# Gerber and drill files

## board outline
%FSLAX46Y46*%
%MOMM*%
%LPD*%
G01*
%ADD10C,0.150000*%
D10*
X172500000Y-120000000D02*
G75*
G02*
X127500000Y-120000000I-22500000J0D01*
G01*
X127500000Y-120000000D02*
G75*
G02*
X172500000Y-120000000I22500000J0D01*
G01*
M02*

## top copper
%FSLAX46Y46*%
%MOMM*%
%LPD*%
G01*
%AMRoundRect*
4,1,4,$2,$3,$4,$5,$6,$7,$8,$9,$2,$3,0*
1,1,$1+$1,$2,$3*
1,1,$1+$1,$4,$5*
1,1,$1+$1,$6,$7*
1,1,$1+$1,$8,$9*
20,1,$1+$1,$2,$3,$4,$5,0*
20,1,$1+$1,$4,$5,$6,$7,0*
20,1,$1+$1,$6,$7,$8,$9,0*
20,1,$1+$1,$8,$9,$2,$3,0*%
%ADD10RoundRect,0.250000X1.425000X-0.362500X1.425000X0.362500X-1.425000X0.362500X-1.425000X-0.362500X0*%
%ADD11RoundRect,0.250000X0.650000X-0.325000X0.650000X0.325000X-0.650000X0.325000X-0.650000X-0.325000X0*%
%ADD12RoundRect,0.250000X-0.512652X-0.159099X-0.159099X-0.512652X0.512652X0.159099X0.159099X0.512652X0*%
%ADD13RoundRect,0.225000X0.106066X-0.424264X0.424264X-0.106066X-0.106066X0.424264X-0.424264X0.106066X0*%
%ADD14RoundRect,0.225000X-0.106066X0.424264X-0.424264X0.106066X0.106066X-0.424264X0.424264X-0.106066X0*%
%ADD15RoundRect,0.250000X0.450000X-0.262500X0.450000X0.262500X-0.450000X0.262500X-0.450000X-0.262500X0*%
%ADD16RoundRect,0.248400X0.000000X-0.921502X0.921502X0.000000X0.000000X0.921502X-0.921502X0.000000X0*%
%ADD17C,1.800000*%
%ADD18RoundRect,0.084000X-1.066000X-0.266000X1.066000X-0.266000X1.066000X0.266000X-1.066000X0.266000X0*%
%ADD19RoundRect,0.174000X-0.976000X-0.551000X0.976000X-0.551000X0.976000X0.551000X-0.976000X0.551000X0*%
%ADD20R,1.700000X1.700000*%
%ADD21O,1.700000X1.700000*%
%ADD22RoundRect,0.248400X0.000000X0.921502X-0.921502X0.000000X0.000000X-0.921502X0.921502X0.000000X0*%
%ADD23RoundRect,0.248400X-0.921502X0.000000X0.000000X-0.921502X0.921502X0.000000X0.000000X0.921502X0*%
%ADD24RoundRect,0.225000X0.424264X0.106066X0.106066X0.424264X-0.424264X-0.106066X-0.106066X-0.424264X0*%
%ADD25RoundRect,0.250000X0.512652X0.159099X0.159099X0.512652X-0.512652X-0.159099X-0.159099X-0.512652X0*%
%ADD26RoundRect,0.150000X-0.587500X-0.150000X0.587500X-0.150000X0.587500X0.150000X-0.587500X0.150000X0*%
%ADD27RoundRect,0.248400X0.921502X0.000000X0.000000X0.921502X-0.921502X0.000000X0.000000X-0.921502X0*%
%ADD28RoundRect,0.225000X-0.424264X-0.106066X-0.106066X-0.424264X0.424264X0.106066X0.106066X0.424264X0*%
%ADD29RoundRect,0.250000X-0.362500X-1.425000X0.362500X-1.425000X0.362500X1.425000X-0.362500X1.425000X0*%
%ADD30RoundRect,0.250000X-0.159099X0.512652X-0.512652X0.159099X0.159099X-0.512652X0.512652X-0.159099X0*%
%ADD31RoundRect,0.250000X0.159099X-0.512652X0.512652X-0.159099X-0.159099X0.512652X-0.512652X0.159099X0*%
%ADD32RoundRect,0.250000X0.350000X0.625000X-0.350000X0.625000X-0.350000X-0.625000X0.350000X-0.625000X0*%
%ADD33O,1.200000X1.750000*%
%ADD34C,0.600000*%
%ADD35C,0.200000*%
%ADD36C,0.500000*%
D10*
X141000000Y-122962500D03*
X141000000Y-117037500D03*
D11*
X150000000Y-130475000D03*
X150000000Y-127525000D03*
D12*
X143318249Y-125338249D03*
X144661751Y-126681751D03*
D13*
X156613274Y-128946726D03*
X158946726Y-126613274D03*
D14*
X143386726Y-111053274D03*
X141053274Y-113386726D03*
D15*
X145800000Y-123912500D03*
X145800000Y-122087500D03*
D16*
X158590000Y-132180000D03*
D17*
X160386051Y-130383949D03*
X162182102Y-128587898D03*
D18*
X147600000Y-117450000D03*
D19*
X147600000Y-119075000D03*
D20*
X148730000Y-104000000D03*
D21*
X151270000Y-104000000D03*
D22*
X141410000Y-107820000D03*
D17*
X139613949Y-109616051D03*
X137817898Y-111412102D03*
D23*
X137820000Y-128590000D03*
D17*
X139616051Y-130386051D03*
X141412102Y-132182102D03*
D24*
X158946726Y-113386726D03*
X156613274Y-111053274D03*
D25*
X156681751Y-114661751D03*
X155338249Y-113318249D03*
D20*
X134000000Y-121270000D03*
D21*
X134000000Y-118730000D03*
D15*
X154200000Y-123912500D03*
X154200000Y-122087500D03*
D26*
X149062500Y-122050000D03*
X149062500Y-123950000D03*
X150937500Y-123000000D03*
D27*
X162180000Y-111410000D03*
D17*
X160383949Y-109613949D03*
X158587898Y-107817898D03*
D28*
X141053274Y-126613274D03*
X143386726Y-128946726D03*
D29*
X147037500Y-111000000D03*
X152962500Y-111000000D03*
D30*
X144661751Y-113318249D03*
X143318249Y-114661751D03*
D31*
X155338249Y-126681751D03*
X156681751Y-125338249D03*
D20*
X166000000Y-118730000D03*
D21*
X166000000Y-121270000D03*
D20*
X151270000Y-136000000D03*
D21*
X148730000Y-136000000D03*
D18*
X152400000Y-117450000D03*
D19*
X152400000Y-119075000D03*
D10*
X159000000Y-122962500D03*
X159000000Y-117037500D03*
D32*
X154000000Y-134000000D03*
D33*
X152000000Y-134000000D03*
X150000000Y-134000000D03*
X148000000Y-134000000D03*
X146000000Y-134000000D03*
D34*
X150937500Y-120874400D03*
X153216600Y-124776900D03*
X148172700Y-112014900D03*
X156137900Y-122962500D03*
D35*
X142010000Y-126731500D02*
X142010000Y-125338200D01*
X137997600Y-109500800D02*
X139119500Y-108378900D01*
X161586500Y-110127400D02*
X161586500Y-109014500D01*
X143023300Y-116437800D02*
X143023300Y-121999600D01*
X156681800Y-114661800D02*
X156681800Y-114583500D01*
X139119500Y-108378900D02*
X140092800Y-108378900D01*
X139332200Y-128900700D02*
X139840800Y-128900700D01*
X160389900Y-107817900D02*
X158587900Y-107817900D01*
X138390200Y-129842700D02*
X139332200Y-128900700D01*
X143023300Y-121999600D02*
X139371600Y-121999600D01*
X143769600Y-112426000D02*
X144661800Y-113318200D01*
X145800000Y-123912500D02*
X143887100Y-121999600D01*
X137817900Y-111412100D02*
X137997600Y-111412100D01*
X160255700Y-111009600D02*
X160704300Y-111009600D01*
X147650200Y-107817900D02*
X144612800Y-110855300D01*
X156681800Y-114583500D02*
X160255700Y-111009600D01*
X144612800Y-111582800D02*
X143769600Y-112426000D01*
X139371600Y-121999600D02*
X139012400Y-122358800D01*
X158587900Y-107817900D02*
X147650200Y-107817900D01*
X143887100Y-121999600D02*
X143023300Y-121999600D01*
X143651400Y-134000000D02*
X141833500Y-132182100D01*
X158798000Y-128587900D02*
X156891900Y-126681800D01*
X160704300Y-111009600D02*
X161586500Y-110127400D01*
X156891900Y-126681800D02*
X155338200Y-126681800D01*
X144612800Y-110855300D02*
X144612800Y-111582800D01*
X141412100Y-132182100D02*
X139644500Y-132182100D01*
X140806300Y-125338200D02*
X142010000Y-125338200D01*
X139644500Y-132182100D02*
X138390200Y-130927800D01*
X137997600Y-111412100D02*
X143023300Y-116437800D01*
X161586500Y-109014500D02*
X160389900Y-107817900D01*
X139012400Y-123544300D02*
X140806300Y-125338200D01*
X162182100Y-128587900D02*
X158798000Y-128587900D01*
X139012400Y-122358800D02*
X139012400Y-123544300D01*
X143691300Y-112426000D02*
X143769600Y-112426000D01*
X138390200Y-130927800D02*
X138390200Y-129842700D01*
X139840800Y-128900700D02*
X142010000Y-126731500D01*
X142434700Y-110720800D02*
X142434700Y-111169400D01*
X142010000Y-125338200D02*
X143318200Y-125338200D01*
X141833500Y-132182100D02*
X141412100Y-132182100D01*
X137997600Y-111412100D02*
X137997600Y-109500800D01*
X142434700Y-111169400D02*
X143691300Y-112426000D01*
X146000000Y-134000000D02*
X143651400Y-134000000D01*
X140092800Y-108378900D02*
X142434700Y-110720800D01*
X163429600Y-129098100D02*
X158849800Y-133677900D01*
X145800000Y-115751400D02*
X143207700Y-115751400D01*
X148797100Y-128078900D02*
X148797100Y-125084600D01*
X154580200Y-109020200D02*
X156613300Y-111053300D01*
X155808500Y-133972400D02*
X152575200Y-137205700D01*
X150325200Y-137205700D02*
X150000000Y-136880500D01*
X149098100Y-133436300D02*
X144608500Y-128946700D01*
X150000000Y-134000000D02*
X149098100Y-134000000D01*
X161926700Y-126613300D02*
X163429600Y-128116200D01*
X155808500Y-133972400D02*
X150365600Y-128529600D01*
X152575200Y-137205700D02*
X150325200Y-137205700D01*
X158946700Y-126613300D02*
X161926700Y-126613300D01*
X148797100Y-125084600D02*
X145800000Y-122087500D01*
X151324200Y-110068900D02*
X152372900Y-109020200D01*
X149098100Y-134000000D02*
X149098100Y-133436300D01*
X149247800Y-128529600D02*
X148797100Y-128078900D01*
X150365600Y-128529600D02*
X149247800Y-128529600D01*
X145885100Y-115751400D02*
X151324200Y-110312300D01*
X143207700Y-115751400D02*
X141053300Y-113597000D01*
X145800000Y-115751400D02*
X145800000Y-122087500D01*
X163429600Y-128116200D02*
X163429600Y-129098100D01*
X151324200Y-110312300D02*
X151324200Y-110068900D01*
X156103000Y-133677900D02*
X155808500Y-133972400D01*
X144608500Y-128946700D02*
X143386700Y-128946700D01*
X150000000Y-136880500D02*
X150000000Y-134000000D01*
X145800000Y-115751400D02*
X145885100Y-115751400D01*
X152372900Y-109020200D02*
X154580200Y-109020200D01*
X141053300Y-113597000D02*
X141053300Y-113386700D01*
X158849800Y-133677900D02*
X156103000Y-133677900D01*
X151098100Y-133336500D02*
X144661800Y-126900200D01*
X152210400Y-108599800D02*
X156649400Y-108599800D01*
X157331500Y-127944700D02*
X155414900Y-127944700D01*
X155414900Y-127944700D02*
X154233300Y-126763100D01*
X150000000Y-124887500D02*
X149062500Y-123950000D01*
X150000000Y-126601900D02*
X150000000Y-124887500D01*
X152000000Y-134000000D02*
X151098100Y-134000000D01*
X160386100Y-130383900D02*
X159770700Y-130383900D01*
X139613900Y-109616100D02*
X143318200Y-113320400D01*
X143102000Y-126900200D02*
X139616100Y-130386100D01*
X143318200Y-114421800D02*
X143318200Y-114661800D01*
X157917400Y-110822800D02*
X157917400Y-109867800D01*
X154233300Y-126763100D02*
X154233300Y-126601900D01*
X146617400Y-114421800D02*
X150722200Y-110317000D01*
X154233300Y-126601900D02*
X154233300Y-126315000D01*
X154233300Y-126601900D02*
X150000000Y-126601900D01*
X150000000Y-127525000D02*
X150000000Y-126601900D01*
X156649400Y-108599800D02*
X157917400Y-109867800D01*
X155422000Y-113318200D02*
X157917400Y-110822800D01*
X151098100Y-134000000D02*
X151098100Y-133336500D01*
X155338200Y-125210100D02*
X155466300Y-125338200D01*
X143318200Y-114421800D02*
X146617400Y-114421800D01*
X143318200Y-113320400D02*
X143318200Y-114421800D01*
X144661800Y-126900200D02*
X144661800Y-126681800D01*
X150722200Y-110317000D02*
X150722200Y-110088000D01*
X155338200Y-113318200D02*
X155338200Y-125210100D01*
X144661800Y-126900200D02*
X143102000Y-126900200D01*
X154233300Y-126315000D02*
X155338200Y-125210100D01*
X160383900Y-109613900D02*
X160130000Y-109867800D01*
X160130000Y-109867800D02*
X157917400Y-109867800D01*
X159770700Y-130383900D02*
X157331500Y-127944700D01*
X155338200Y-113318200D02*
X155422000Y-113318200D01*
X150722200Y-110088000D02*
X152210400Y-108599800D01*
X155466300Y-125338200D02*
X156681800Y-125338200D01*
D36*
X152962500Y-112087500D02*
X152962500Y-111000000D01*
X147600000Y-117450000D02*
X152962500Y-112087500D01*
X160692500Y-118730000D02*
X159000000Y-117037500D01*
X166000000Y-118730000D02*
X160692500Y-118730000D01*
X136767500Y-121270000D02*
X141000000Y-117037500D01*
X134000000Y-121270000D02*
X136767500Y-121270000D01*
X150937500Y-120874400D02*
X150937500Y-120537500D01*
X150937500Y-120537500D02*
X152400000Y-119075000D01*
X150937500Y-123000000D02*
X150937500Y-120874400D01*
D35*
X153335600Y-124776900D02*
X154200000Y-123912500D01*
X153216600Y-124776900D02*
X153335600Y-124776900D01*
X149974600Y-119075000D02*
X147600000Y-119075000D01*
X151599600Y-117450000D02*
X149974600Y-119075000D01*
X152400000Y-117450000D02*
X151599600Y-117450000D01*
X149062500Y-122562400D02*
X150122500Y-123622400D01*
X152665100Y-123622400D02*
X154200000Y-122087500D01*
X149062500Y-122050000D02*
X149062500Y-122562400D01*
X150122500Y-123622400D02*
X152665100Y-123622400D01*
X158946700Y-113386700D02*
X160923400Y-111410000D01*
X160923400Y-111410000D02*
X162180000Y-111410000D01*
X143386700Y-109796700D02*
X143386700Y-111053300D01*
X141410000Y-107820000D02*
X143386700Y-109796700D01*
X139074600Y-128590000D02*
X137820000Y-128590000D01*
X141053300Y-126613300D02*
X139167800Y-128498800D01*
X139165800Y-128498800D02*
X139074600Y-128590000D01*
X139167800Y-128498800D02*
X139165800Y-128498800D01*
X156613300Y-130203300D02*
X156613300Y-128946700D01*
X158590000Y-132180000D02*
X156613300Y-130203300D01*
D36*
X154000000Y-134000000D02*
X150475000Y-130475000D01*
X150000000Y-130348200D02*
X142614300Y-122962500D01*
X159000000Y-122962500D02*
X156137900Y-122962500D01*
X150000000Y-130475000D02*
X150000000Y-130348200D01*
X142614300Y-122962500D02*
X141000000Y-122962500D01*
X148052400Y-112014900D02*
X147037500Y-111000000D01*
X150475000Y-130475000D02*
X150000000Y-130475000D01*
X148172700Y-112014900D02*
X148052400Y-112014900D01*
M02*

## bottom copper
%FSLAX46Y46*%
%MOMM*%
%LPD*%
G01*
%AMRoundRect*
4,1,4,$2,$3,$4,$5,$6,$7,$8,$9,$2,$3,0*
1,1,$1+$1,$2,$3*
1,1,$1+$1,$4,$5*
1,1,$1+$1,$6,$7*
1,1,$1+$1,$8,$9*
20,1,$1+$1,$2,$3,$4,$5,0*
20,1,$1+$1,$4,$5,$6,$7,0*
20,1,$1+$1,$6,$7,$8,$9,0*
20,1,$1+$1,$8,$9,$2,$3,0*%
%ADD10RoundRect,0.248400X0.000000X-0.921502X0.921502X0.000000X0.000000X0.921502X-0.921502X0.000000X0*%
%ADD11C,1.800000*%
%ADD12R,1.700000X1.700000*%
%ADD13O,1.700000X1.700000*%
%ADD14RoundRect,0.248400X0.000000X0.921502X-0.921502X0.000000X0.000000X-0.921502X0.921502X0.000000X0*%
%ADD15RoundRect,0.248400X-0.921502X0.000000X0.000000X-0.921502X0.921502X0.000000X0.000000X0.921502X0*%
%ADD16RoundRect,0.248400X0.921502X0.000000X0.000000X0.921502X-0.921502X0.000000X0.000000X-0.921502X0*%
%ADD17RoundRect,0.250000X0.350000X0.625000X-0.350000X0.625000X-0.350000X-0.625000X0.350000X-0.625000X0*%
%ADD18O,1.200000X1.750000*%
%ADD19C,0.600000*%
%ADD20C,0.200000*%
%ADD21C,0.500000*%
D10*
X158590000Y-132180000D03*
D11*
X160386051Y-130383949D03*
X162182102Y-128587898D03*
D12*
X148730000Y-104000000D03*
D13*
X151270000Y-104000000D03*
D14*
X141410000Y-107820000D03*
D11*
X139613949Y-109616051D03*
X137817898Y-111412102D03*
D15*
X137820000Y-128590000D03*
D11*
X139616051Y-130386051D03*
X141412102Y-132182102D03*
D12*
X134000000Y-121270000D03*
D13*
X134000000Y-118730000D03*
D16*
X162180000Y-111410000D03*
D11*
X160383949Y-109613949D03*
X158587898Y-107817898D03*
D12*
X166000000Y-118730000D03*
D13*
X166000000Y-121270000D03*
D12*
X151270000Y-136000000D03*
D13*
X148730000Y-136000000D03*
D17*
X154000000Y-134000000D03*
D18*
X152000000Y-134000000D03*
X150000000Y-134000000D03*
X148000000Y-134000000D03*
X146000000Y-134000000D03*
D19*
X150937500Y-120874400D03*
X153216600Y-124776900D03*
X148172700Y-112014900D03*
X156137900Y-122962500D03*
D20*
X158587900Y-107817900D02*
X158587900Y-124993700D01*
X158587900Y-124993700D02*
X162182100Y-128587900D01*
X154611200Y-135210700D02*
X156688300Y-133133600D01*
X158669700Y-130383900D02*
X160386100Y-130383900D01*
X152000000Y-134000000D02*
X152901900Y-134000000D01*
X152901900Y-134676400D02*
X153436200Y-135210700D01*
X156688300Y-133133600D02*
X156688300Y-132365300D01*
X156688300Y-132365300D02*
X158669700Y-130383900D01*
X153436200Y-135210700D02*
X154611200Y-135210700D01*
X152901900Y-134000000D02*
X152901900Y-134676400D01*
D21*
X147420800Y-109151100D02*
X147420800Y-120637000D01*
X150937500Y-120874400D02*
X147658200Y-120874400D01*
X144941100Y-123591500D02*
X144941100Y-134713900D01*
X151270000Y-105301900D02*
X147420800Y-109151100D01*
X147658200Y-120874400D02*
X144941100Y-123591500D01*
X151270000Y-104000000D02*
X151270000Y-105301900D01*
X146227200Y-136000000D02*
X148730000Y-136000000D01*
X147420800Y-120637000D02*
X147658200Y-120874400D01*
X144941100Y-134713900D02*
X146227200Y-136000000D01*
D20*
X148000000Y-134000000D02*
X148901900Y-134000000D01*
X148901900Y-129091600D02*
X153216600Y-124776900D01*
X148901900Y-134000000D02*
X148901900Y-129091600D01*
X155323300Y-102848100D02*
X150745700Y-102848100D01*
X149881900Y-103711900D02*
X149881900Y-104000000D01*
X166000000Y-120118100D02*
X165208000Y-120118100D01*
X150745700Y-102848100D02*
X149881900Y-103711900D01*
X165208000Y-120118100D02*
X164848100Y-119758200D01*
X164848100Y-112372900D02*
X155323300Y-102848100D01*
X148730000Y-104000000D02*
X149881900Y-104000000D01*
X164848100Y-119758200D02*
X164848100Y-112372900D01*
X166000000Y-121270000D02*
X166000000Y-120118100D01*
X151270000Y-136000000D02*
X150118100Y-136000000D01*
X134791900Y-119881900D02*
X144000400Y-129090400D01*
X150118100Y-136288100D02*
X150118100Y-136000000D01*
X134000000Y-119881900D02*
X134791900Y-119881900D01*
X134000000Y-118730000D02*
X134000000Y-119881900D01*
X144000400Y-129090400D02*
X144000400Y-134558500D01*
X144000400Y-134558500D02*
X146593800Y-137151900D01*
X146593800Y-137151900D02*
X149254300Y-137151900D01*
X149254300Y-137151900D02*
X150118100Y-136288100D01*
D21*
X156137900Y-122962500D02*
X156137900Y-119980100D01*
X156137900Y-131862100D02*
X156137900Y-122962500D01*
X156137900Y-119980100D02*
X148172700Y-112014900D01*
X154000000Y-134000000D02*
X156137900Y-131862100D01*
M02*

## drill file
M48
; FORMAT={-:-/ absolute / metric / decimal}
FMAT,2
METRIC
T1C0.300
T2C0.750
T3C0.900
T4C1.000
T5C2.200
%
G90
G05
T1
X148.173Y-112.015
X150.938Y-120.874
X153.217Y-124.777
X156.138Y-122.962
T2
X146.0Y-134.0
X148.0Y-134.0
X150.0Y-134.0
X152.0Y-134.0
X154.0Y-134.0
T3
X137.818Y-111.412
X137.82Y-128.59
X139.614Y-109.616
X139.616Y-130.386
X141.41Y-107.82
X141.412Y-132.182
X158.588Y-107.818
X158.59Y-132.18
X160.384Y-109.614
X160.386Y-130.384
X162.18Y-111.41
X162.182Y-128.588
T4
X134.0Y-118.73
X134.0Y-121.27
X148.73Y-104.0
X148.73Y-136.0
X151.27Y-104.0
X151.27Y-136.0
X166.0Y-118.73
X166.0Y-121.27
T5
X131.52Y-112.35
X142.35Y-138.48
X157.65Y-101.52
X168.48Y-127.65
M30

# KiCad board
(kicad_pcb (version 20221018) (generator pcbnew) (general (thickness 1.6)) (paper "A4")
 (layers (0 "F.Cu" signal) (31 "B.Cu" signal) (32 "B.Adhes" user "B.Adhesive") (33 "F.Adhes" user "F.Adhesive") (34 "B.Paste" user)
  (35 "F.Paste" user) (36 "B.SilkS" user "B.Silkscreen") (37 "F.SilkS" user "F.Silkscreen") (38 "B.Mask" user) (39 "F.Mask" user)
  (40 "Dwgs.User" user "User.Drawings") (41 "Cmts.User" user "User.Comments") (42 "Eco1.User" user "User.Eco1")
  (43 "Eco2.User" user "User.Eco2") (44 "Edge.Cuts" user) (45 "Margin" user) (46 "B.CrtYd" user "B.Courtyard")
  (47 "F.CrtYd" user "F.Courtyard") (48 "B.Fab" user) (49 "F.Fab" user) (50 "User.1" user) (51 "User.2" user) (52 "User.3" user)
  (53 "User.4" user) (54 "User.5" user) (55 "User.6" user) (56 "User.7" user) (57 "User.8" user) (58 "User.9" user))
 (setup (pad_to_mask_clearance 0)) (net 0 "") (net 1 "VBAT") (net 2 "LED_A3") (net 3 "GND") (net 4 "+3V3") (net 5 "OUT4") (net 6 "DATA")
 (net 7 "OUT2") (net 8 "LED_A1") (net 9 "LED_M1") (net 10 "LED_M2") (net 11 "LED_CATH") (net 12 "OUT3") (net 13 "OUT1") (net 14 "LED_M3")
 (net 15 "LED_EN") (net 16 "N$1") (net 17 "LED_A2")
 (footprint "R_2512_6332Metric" (layer "F.Cu") (at 141 120 90)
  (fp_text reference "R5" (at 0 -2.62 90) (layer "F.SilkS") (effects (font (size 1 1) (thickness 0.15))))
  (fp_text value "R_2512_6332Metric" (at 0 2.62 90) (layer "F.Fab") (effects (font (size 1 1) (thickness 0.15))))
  (pad "1" smd roundrect (at -2.9625 0 90) (size 1.225 3.35) (layers "F.Cu" "F.Paste" "F.Mask") (roundrect_rratio 0.204082) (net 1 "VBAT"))
  (pad "2" smd roundrect (at 2.9625 0 90) (size 1.225 3.35) (layers "F.Cu" "F.Paste" "F.Mask") (roundrect_rratio 0.204082) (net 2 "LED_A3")))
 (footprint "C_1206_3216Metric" (layer "F.Cu") (at 150 129 90)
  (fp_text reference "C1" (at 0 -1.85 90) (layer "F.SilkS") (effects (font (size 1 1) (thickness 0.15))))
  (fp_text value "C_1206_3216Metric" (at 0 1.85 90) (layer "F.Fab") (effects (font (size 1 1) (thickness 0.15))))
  (pad "1" smd roundrect (at -1.475 0 90) (size 1.15 1.8) (layers "F.Cu" "F.Paste" "F.Mask") (roundrect_rratio 0.217391) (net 1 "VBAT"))
  (pad "2" smd roundrect (at 1.475 0 90) (size 1.15 1.8) (layers "F.Cu" "F.Paste" "F.Mask") (roundrect_rratio 0.217391) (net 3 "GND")))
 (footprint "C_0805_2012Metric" (layer "F.Cu") (at 143.99 126.01 -45)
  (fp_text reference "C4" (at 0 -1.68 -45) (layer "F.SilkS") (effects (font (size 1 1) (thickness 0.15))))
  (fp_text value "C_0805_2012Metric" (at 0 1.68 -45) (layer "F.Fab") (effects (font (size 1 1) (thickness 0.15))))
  (pad "1" smd roundrect (at -0.95 0 315) (size 1 1.45) (layers "F.Cu" "F.Paste" "F.Mask") (roundrect_rratio 0.25) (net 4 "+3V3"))
  (pad "2" smd roundrect (at 0.95 0 315) (size 1 1.45) (layers "F.Cu" "F.Paste" "F.Mask") (roundrect_rratio 0.25) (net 3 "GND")))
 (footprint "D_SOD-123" (layer "F.Cu") (at 157.78 127.78 45)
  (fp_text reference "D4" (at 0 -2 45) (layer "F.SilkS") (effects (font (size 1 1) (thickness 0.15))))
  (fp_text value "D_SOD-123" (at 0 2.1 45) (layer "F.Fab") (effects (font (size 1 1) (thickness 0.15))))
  (pad "1" smd roundrect (at -1.65 0 45) (size 0.9 1.2) (layers "F.Cu" "F.Paste" "F.Mask") (roundrect_rratio 0.25) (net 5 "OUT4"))
  (pad "2" smd roundrect (at 1.65 0 45) (size 0.9 1.2) (layers "F.Cu" "F.Paste" "F.Mask") (roundrect_rratio 0.25) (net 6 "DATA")))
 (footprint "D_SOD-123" (layer "F.Cu") (at 142.22 112.22 -135)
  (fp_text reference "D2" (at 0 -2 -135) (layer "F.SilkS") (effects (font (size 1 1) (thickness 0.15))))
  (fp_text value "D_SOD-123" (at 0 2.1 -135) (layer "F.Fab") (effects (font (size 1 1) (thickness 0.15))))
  (pad "1" smd roundrect (at -1.65 0 225) (size 0.9 1.2) (layers "F.Cu" "F.Paste" "F.Mask") (roundrect_rratio 0.25) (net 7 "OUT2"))
  (pad "2" smd roundrect (at 1.65 0 225) (size 0.9 1.2) (layers "F.Cu" "F.Paste" "F.Mask") (roundrect_rratio 0.25) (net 6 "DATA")))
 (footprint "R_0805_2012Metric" (layer "F.Cu") (at 145.8 123 90)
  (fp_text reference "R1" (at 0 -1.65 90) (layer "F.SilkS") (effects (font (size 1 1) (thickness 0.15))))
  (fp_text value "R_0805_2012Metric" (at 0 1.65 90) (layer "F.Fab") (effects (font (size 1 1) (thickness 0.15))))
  (pad "1" smd roundrect (at -0.9125 0 90) (size 1.025 1.4) (layers "F.Cu" "F.Paste" "F.Mask") (roundrect_rratio 0.243902) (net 4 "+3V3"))
  (pad "2" smd roundrect (at 0.9125 0 90) (size 1.025 1.4) (layers "F.Cu" "F.Paste" "F.Mask") (roundrect_rratio 0.243902) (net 6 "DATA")))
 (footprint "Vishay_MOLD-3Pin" (layer "F.Cu") (at 158.59 132.18 45)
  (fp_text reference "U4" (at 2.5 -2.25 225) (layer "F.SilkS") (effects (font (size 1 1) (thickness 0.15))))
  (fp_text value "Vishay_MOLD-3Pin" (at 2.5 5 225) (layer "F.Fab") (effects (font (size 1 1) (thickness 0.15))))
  (pad "1" thru_hole roundrect (at 0 0 45) (size 1.8 1.8) (drill 0.9) (layers "*.Cu" "*.Mask") (roundrect_rratio 0.138) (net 5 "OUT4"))
  (pad "2" thru_hole circle (at 2.54 0 45) (size 1.8 1.8) (drill 0.9) (layers "*.Cu" "*.Mask") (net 3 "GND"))
  (pad "3" thru_hole circle (at 5.08 0 45) (size 1.8 1.8) (drill 0.9) (layers "*.Cu" "*.Mask") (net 4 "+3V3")))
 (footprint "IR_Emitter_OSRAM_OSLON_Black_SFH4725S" (layer "F.Cu") (at 147.6 118.5)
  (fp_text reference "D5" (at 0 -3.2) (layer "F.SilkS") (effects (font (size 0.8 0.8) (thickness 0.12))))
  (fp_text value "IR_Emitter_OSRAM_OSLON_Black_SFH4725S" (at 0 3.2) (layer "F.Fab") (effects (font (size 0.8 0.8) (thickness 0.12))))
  (pad "1" smd roundrect (at 0 -1.05) (size 2.3 0.7) (layers "F.Cu" "F.Paste" "F.Mask") (roundrect_rratio 0.12) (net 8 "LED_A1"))
  (pad "2" smd roundrect (at 0 0.575) (size 2.3 1.45) (layers "F.Cu" "F.Paste" "F.Mask") (roundrect_rratio 0.12) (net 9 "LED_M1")))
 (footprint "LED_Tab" (layer "F.Cu") (at 148.73 104 90)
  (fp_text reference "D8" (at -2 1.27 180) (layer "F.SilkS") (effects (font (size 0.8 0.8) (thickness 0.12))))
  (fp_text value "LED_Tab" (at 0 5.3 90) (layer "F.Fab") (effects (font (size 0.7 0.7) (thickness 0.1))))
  (pad "1" thru_hole rect (at 0 0 90) (size 1.7 1.7) (drill 1) (layers "*.Cu" "*.Mask") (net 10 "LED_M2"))
  (pad "2" thru_hole oval (at 0 2.54 90) (size 1.7 1.7) (drill 1) (layers "*.Cu" "*.Mask") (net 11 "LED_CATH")))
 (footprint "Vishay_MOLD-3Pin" (layer "F.Cu") (at 141.41 107.82 -135)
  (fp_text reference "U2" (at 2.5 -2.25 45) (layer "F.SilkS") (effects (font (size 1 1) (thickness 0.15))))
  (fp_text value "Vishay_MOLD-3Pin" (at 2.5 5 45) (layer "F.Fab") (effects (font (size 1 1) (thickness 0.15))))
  (pad "1" thru_hole roundrect (at 0 0 225) (size 1.8 1.8) (drill 0.9) (layers "*.Cu" "*.Mask") (roundrect_rratio 0.138) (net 7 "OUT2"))
  (pad "2" thru_hole circle (at 2.54 0 225) (size 1.8 1.8) (drill 0.9) (layers "*.Cu" "*.Mask") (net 3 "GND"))
  (pad "3" thru_hole circle (at 5.08 0 225) (size 1.8 1.8) (drill 0.9) (layers "*.Cu" "*.Mask") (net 4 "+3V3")))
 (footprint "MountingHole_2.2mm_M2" (layer "F.Cu") (at 131.52 112.35)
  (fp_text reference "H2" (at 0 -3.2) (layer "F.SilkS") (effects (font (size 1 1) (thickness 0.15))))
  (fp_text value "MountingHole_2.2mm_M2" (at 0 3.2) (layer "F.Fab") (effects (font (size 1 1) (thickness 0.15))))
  (pad "" np_thru_hole circle (at 0 0) (size 2.2 2.2) (drill 2.2) (layers "*.Cu" "*.Mask")))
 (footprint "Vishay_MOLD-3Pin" (layer "F.Cu") (at 137.82 128.59 -45)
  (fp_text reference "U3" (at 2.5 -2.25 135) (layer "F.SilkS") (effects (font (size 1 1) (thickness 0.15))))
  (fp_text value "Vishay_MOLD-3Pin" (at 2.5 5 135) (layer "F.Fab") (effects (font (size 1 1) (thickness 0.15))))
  (pad "1" thru_hole roundrect (at 0 0 315) (size 1.8 1.8) (drill 0.9) (layers "*.Cu" "*.Mask") (roundrect_rratio 0.138) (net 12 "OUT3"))
  (pad "2" thru_hole circle (at 2.54 0 315) (size 1.8 1.8) (drill 0.9) (layers "*.Cu" "*.Mask") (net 3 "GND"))
  (pad "3" thru_hole circle (at 5.08 0 315) (size 1.8 1.8) (drill 0.9) (layers "*.Cu" "*.Mask") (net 4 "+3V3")))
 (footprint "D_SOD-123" (layer "F.Cu") (at 157.78 112.22 135)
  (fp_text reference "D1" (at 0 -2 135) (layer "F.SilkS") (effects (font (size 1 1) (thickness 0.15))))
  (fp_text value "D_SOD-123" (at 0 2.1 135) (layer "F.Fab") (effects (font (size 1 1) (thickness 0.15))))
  (pad "1" smd roundrect (at -1.65 0 135) (size 0.9 1.2) (layers "F.Cu" "F.Paste" "F.Mask") (roundrect_rratio 0.25) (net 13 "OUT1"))
  (pad "2" smd roundrect (at 1.65 0 135) (size 0.9 1.2) (layers "F.Cu" "F.Paste" "F.Mask") (roundrect_rratio 0.25) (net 6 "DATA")))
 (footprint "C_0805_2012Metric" (layer "F.Cu") (at 156.01 113.99 135)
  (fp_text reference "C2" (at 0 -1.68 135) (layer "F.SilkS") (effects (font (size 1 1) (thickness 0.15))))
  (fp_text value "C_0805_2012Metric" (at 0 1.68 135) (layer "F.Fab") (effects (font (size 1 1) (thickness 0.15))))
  (pad "1" smd roundrect (at -0.95 0 135) (size 1 1.45) (layers "F.Cu" "F.Paste" "F.Mask") (roundrect_rratio 0.25) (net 4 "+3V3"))
  (pad "2" smd roundrect (at 0.95 0 135) (size 1 1.45) (layers "F.Cu" "F.Paste" "F.Mask") (roundrect_rratio 0.25) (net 3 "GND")))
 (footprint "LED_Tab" (layer "F.Cu") (at 134 121.27 180)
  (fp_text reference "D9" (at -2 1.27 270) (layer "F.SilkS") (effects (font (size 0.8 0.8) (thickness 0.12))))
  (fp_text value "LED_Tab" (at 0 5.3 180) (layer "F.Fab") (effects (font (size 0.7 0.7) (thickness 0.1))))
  (pad "1" thru_hole rect (at 0 0 180) (size 1.7 1.7) (drill 1) (layers "*.Cu" "*.Mask") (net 2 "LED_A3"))
  (pad "2" thru_hole oval (at 0 2.54 180) (size 1.7 1.7) (drill 1) (layers "*.Cu" "*.Mask") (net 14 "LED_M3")))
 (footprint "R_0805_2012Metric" (layer "F.Cu") (at 154.2 123 90)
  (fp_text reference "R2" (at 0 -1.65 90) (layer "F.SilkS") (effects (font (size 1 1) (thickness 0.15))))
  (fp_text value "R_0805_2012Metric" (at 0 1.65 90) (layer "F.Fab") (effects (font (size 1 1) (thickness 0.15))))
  (pad "1" smd roundrect (at -0.9125 0 90) (size 1.025 1.4) (layers "F.Cu" "F.Paste" "F.Mask") (roundrect_rratio 0.243902) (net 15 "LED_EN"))
  (pad "2" smd roundrect (at 0.9125 0 90) (size 1.025 1.4) (layers "F.Cu" "F.Paste" "F.Mask") (roundrect_rratio 0.243902) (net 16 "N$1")))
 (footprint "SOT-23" (layer "F.Cu") (at 150 123)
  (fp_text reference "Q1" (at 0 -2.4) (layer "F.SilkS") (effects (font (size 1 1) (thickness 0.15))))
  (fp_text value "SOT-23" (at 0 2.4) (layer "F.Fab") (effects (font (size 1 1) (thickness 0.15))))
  (pad "1" smd roundrect (at -0.9375 -0.95) (size 1.475 0.6) (layers "F.Cu" "F.Paste" "F.Mask") (roundrect_rratio 0.25) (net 16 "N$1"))
  (pad "2" smd roundrect (at -0.9375 0.95) (size 1.475 0.6) (layers "F.Cu" "F.Paste" "F.Mask") (roundrect_rratio 0.25) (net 3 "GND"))
  (pad "3" smd roundrect (at 0.9375 0) (size 1.475 0.6) (layers "F.Cu" "F.Paste" "F.Mask") (roundrect_rratio 0.25) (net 11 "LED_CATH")))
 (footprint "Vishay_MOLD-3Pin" (layer "F.Cu") (at 162.18 111.41 135)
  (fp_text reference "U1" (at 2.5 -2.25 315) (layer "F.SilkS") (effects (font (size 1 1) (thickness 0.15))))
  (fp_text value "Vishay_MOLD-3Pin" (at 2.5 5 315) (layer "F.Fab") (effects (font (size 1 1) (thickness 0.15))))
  (pad "1" thru_hole roundrect (at 0 0 135) (size 1.8 1.8) (drill 0.9) (layers "*.Cu" "*.Mask") (roundrect_rratio 0.138) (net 13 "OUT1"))
  (pad "2" thru_hole circle (at 2.54 0 135) (size 1.8 1.8) (drill 0.9) (layers "*.Cu" "*.Mask") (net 3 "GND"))
  (pad "3" thru_hole circle (at 5.08 0 135) (size 1.8 1.8) (drill 0.9) (layers "*.Cu" "*.Mask") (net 4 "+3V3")))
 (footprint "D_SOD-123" (layer "F.Cu") (at 142.22 127.78 -45)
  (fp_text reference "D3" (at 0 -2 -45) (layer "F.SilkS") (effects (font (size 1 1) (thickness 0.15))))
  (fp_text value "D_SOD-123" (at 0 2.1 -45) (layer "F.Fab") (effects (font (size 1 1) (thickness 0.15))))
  (pad "1" smd roundrect (at -1.65 0 315) (size 0.9 1.2) (layers "F.Cu" "F.Paste" "F.Mask") (roundrect_rratio 0.25) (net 12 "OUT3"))
  (pad "2" smd roundrect (at 1.65 0 315) (size 0.9 1.2) (layers "F.Cu" "F.Paste" "F.Mask") (roundrect_rratio 0.25) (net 6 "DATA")))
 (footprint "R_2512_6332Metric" (layer "F.Cu") (at 150 111)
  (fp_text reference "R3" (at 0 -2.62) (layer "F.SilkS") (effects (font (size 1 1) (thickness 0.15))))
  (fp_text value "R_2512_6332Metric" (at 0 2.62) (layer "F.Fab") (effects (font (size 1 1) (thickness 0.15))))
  (pad "1" smd roundrect (at -2.9625 0) (size 1.225 3.35) (layers "F.Cu" "F.Paste" "F.Mask") (roundrect_rratio 0.204082) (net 1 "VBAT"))
  (pad "2" smd roundrect (at 2.9625 0) (size 1.225 3.35) (layers "F.Cu" "F.Paste" "F.Mask") (roundrect_rratio 0.204082) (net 8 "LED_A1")))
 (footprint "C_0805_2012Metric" (layer "F.Cu") (at 143.99 113.99 -135)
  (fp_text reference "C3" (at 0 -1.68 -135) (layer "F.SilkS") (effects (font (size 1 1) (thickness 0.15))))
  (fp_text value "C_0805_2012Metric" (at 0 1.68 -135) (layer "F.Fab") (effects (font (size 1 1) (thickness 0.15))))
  (pad "1" smd roundrect (at -0.95 0 225) (size 1 1.45) (layers "F.Cu" "F.Paste" "F.Mask") (roundrect_rratio 0.25) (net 4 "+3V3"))
  (pad "2" smd roundrect (at 0.95 0 225) (size 1 1.45) (layers "F.Cu" "F.Paste" "F.Mask") (roundrect_rratio 0.25) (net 3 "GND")))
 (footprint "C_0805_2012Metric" (layer "F.Cu") (at 156.01 126.01 45)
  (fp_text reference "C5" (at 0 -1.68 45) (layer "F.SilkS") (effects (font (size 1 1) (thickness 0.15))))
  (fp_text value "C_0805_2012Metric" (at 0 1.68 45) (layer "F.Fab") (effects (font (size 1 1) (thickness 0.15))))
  (pad "1" smd roundrect (at -0.95 0 45) (size 1 1.45) (layers "F.Cu" "F.Paste" "F.Mask") (roundrect_rratio 0.25) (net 4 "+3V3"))
  (pad "2" smd roundrect (at 0.95 0 45) (size 1 1.45) (layers "F.Cu" "F.Paste" "F.Mask") (roundrect_rratio 0.25) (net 3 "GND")))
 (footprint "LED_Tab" (layer "F.Cu") (at 166 118.73)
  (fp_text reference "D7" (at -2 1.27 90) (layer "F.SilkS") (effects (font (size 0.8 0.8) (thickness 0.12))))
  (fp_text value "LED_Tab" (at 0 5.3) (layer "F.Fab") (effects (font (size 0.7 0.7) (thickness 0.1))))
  (pad "1" thru_hole rect (at 0 0) (size 1.7 1.7) (drill 1) (layers "*.Cu" "*.Mask") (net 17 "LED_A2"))
  (pad "2" thru_hole oval (at 0 2.54) (size 1.7 1.7) (drill 1) (layers "*.Cu" "*.Mask") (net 10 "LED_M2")))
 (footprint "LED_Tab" (layer "F.Cu") (at 151.27 136 -90)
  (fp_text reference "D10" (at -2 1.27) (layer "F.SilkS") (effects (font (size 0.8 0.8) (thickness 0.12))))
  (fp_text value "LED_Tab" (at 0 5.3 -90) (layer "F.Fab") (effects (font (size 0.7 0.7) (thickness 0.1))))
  (pad "1" thru_hole rect (at 0 0 270) (size 1.7 1.7) (drill 1) (layers "*.Cu" "*.Mask") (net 14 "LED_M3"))
  (pad "2" thru_hole oval (at 0 2.54 270) (size 1.7 1.7) (drill 1) (layers "*.Cu" "*.Mask") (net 11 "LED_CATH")))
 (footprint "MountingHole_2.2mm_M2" (layer "F.Cu") (at 168.48 127.65)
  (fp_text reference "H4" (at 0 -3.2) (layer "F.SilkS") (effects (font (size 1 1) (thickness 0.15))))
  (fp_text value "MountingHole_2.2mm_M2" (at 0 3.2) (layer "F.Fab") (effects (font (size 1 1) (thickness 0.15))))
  (pad "" np_thru_hole circle (at 0 0) (size 2.2 2.2) (drill 2.2) (layers "*.Cu" "*.Mask")))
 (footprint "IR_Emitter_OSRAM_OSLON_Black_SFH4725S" (layer "F.Cu") (at 152.4 118.5)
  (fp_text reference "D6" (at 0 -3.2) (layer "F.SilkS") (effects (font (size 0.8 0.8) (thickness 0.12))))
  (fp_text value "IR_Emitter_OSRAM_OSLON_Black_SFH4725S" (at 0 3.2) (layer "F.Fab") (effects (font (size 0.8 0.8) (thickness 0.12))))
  (pad "1" smd roundrect (at 0 -1.05) (size 2.3 0.7) (layers "F.Cu" "F.Paste" "F.Mask") (roundrect_rratio 0.12) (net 9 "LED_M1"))
  (pad "2" smd roundrect (at 0 0.575) (size 2.3 1.45) (layers "F.Cu" "F.Paste" "F.Mask") (roundrect_rratio 0.12) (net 11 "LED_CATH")))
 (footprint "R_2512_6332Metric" (layer "F.Cu") (at 159 120 90)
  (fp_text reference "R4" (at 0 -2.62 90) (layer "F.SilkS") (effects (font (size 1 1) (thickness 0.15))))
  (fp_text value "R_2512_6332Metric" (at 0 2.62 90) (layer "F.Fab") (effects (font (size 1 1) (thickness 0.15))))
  (pad "1" smd roundrect (at -2.9625 0 90) (size 1.225 3.35) (layers "F.Cu" "F.Paste" "F.Mask") (roundrect_rratio 0.204082) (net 1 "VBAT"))
  (pad "2" smd roundrect (at 2.9625 0 90) (size 1.225 3.35) (layers "F.Cu" "F.Paste" "F.Mask") (roundrect_rratio 0.204082) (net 17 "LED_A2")))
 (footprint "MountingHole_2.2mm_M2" (layer "F.Cu") (at 142.35 138.48)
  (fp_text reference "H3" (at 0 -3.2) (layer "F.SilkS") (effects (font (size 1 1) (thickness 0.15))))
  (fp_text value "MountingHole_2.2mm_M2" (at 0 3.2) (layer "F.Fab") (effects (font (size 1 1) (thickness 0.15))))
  (pad "" np_thru_hole circle (at 0 0) (size 2.2 2.2) (drill 2.2) (layers "*.Cu" "*.Mask")))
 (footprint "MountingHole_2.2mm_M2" (layer "F.Cu") (at 157.65 101.52)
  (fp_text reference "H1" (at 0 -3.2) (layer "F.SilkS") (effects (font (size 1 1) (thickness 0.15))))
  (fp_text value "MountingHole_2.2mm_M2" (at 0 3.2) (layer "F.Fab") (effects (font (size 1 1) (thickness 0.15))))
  (pad "" np_thru_hole circle (at 0 0) (size 2.2 2.2) (drill 2.2) (layers "*.Cu" "*.Mask")))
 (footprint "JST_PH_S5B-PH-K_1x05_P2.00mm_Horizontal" (layer "B.Cu") (at 154 134 180)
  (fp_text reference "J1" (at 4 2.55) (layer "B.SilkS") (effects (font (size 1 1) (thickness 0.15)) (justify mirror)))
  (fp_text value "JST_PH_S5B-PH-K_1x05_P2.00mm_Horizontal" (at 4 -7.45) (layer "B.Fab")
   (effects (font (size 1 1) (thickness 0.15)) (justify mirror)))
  (pad "1" thru_hole roundrect (at 0 0 180) (size 1.2 1.75) (drill 0.75) (layers "*.Cu" "*.Mask") (roundrect_rratio 0.208333) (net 1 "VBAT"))
  (pad "2" thru_hole oval (at 2 0 180) (size 1.2 1.75) (drill 0.75) (layers "*.Cu" "*.Mask") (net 3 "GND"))
  (pad "3" thru_hole oval (at 4 0 180) (size 1.2 1.75) (drill 0.75) (layers "*.Cu" "*.Mask") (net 6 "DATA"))
  (pad "4" thru_hole oval (at 6 0 180) (size 1.2 1.75) (drill 0.75) (layers "*.Cu" "*.Mask") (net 15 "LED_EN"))
  (pad "5" thru_hole oval (at 8 0 180) (size 1.2 1.75) (drill 0.75) (layers "*.Cu" "*.Mask") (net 4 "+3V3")))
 (gr_circle (center 150 120) (end 172.5 120) (stroke (width 0.15) (type default)) (fill none) (layer "Edge.Cuts"))
 (segment (start 142.01 126.7315) (end 142.01 125.3382) (width 0.2) (layer "F.Cu") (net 4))
 (segment (start 137.9976 109.5008) (end 139.1195 108.3789) (width 0.2) (layer "F.Cu") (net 4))
 (segment (start 161.5865 110.1274) (end 161.5865 109.0145) (width 0.2) (layer "F.Cu") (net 4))
 (segment (start 143.0233 116.4378) (end 143.0233 121.9996) (width 0.2) (layer "F.Cu") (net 4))
 (segment (start 156.6818 114.6618) (end 156.6818 114.5835) (width 0.2) (layer "F.Cu") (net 4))
 (segment (start 139.1195 108.3789) (end 140.0928 108.3789) (width 0.2) (layer "F.Cu") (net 4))
 (segment (start 139.3322 128.9007) (end 139.8408 128.9007) (width 0.2) (layer "F.Cu") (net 4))
 (segment (start 160.3899 107.8179) (end 158.5879 107.8179) (width 0.2) (layer "F.Cu") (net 4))
 (segment (start 138.3902 129.8427) (end 139.3322 128.9007) (width 0.2) (layer "F.Cu") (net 4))
 (segment (start 143.0233 121.9996) (end 139.3716 121.9996) (width 0.2) (layer "F.Cu") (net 4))
 (segment (start 143.7696 112.426) (end 144.6618 113.3182) (width 0.2) (layer "F.Cu") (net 4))
 (segment (start 145.8 123.9125) (end 143.8871 121.9996) (width 0.2) (layer "F.Cu") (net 4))
 (segment (start 137.8179 111.4121) (end 137.9976 111.4121) (width 0.2) (layer "F.Cu") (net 4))
 (segment (start 160.2557 111.0096) (end 160.7043 111.0096) (width 0.2) (layer "F.Cu") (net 4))
 (segment (start 147.6502 107.8179) (end 144.6128 110.8553) (width 0.2) (layer "F.Cu") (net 4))
 (segment (start 156.6818 114.5835) (end 160.2557 111.0096) (width 0.2) (layer "F.Cu") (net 4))
 (segment (start 144.6128 111.5828) (end 143.7696 112.426) (width 0.2) (layer "F.Cu") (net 4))
 (segment (start 139.3716 121.9996) (end 139.0124 122.3588) (width 0.2) (layer "F.Cu") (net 4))
 (segment (start 158.5879 107.8179) (end 147.6502 107.8179) (width 0.2) (layer "F.Cu") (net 4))
 (segment (start 143.8871 121.9996) (end 143.0233 121.9996) (width 0.2) (layer "F.Cu") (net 4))
 (segment (start 143.6514 134) (end 141.8335 132.1821) (width 0.2) (layer "F.Cu") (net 4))
 (segment (start 158.798 128.5879) (end 156.8919 126.6818) (width 0.2) (layer "F.Cu") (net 4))
 (segment (start 160.7043 111.0096) (end 161.5865 110.1274) (width 0.2) (layer "F.Cu") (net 4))
 (segment (start 156.8919 126.6818) (end 155.3382 126.6818) (width 0.2) (layer "F.Cu") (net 4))
 (segment (start 144.6128 110.8553) (end 144.6128 111.5828) (width 0.2) (layer "F.Cu") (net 4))
 (segment (start 141.4121 132.1821) (end 139.6445 132.1821) (width 0.2) (layer "F.Cu") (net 4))
 (segment (start 140.8063 125.3382) (end 142.01 125.3382) (width 0.2) (layer "F.Cu") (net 4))
 (segment (start 139.6445 132.1821) (end 138.3902 130.9278) (width 0.2) (layer "F.Cu") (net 4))
 (segment (start 137.9976 111.4121) (end 143.0233 116.4378) (width 0.2) (layer "F.Cu") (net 4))
 (segment (start 161.5865 109.0145) (end 160.3899 107.8179) (width 0.2) (layer "F.Cu") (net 4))
 (segment (start 139.0124 123.5443) (end 140.8063 125.3382) (width 0.2) (layer "F.Cu") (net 4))
 (segment (start 162.1821 128.5879) (end 158.798 128.5879) (width 0.2) (layer "F.Cu") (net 4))
 (segment (start 139.0124 122.3588) (end 139.0124 123.5443) (width 0.2) (layer "F.Cu") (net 4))
 (segment (start 143.6913 112.426) (end 143.7696 112.426) (width 0.2) (layer "F.Cu") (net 4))
 (segment (start 138.3902 130.9278) (end 138.3902 129.8427) (width 0.2) (layer "F.Cu") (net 4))
 (segment (start 139.8408 128.9007) (end 142.01 126.7315) (width 0.2) (layer "F.Cu") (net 4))
 (segment (start 142.4347 110.7208) (end 142.4347 111.1694) (width 0.2) (layer "F.Cu") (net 4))
 (segment (start 142.01 125.3382) (end 143.3182 125.3382) (width 0.2) (layer "F.Cu") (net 4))
 (segment (start 141.8335 132.1821) (end 141.4121 132.1821) (width 0.2) (layer "F.Cu") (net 4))
 (segment (start 137.9976 111.4121) (end 137.9976 109.5008) (width 0.2) (layer "F.Cu") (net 4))
 (segment (start 142.4347 111.1694) (end 143.6913 112.426) (width 0.2) (layer "F.Cu") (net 4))
 (segment (start 146 134) (end 143.6514 134) (width 0.2) (layer "F.Cu") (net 4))
 (segment (start 140.0928 108.3789) (end 142.4347 110.7208) (width 0.2) (layer "F.Cu") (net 4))
 (segment (start 158.5879 107.8179) (end 158.5879 124.9937) (width 0.2) (layer "B.Cu") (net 4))
 (segment (start 158.5879 124.9937) (end 162.1821 128.5879) (width 0.2) (layer "B.Cu") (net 4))
 (segment (start 163.4296 129.0981) (end 158.8498 133.6779) (width 0.2) (layer "F.Cu") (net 6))
 (segment (start 145.8 115.7514) (end 143.2077 115.7514) (width 0.2) (layer "F.Cu") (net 6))
 (segment (start 148.7971 128.0789) (end 148.7971 125.0846) (width 0.2) (layer "F.Cu") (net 6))
 (segment (start 154.5802 109.0202) (end 156.6133 111.0533) (width 0.2) (layer "F.Cu") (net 6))
 (segment (start 155.8085 133.9724) (end 152.5752 137.2057) (width 0.2) (layer "F.Cu") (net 6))
 (segment (start 150.3252 137.2057) (end 150 136.8805) (width 0.2) (layer "F.Cu") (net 6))
 (segment (start 149.0981 133.4363) (end 144.6085 128.9467) (width 0.2) (layer "F.Cu") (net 6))
 (segment (start 150 134) (end 149.0981 134) (width 0.2) (layer "F.Cu") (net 6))
 (segment (start 161.9267 126.6133) (end 163.4296 128.1162) (width 0.2) (layer "F.Cu") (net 6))
 (segment (start 155.8085 133.9724) (end 150.3656 128.5296) (width 0.2) (layer "F.Cu") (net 6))
 (segment (start 152.5752 137.2057) (end 150.3252 137.2057) (width 0.2) (layer "F.Cu") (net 6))
 (segment (start 158.9467 126.6133) (end 161.9267 126.6133) (width 0.2) (layer "F.Cu") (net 6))
 (segment (start 148.7971 125.0846) (end 145.8 122.0875) (width 0.2) (layer "F.Cu") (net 6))
 (segment (start 151.3242 110.0689) (end 152.3729 109.0202) (width 0.2) (layer "F.Cu") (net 6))
 (segment (start 149.0981 134) (end 149.0981 133.4363) (width 0.2) (layer "F.Cu") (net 6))
 (segment (start 149.2478 128.5296) (end 148.7971 128.0789) (width 0.2) (layer "F.Cu") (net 6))
 (segment (start 150.3656 128.5296) (end 149.2478 128.5296) (width 0.2) (layer "F.Cu") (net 6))
 (segment (start 145.8851 115.7514) (end 151.3242 110.3123) (width 0.2) (layer "F.Cu") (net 6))
 (segment (start 143.2077 115.7514) (end 141.0533 113.597) (width 0.2) (layer "F.Cu") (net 6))
 (segment (start 145.8 115.7514) (end 145.8 122.0875) (width 0.2) (layer "F.Cu") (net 6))
 (segment (start 163.4296 128.1162) (end 163.4296 129.0981) (width 0.2) (layer "F.Cu") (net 6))
 (segment (start 151.3242 110.3123) (end 151.3242 110.0689) (width 0.2) (layer "F.Cu") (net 6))
 (segment (start 156.103 133.6779) (end 155.8085 133.9724) (width 0.2) (layer "F.Cu") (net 6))
 (segment (start 144.6085 128.9467) (end 143.3867 128.9467) (width 0.2) (layer "F.Cu") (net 6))
 (segment (start 150 136.8805) (end 150 134) (width 0.2) (layer "F.Cu") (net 6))
 (segment (start 145.8 115.7514) (end 145.8851 115.7514) (width 0.2) (layer "F.Cu") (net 6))
 (segment (start 152.3729 109.0202) (end 154.5802 109.0202) (width 0.2) (layer "F.Cu") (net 6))
 (segment (start 141.0533 113.597) (end 141.0533 113.3867) (width 0.2) (layer "F.Cu") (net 6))
 (segment (start 158.8498 133.6779) (end 156.103 133.6779) (width 0.2) (layer "F.Cu") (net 6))
 (segment (start 151.0981 133.3365) (end 144.6618 126.9002) (width 0.2) (layer "F.Cu") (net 3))
 (segment (start 152.2104 108.5998) (end 156.6494 108.5998) (width 0.2) (layer "F.Cu") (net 3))
 (segment (start 157.3315 127.9447) (end 155.4149 127.9447) (width 0.2) (layer "F.Cu") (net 3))
 (segment (start 155.4149 127.9447) (end 154.2333 126.7631) (width 0.2) (layer "F.Cu") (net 3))
 (segment (start 150 124.8875) (end 149.0625 123.95) (width 0.2) (layer "F.Cu") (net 3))
 (segment (start 150 126.6019) (end 150 124.8875) (width 0.2) (layer "F.Cu") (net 3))
 (segment (start 152 134) (end 151.0981 134) (width 0.2) (layer "F.Cu") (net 3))
 (segment (start 160.3861 130.3839) (end 159.7707 130.3839) (width 0.2) (layer "F.Cu") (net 3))
 (segment (start 139.6139 109.6161) (end 143.3182 113.3204) (width 0.2) (layer "F.Cu") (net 3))
 (segment (start 143.102 126.9002) (end 139.6161 130.3861) (width 0.2) (layer "F.Cu") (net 3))
 (segment (start 143.3182 114.4218) (end 143.3182 114.6618) (width 0.2) (layer "F.Cu") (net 3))
 (segment (start 157.9174 110.8228) (end 157.9174 109.8678) (width 0.2) (layer "F.Cu") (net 3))
 (segment (start 154.2333 126.7631) (end 154.2333 126.6019) (width 0.2) (layer "F.Cu") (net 3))
 (segment (start 146.6174 114.4218) (end 150.7222 110.317) (width 0.2) (layer "F.Cu") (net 3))
 (segment (start 154.2333 126.6019) (end 154.2333 126.315) (width 0.2) (layer "F.Cu") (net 3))
 (segment (start 154.2333 126.6019) (end 150 126.6019) (width 0.2) (layer "F.Cu") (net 3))
 (segment (start 150 127.525) (end 150 126.6019) (width 0.2) (layer "F.Cu") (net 3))
 (segment (start 156.6494 108.5998) (end 157.9174 109.8678) (width 0.2) (layer "F.Cu") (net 3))
 (segment (start 155.422 113.3182) (end 157.9174 110.8228) (width 0.2) (layer "F.Cu") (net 3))
 (segment (start 151.0981 134) (end 151.0981 133.3365) (width 0.2) (layer "F.Cu") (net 3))
 (segment (start 155.3382 125.2101) (end 155.4663 125.3382) (width 0.2) (layer "F.Cu") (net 3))
 (segment (start 143.3182 114.4218) (end 146.6174 114.4218) (width 0.2) (layer "F.Cu") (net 3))
 (segment (start 143.3182 113.3204) (end 143.3182 114.4218) (width 0.2) (layer "F.Cu") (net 3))
 (segment (start 144.6618 126.9002) (end 144.6618 126.6818) (width 0.2) (layer "F.Cu") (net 3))
 (segment (start 150.7222 110.317) (end 150.7222 110.088) (width 0.2) (layer "F.Cu") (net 3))
 (segment (start 155.3382 113.3182) (end 155.3382 125.2101) (width 0.2) (layer "F.Cu") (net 3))
 (segment (start 144.6618 126.9002) (end 143.102 126.9002) (width 0.2) (layer "F.Cu") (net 3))
 (segment (start 154.2333 126.315) (end 155.3382 125.2101) (width 0.2) (layer "F.Cu") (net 3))
 (segment (start 160.3839 109.6139) (end 160.13 109.8678) (width 0.2) (layer "F.Cu") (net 3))
 (segment (start 160.13 109.8678) (end 157.9174 109.8678) (width 0.2) (layer "F.Cu") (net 3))
 (segment (start 159.7707 130.3839) (end 157.3315 127.9447) (width 0.2) (layer "F.Cu") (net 3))
 (segment (start 155.3382 113.3182) (end 155.422 113.3182) (width 0.2) (layer "F.Cu") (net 3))
 (segment (start 150.7222 110.088) (end 152.2104 108.5998) (width 0.2) (layer "F.Cu") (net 3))
 (segment (start 155.4663 125.3382) (end 156.6818 125.3382) (width 0.2) (layer "F.Cu") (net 3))
 (segment (start 154.6112 135.2107) (end 156.6883 133.1336) (width 0.2) (layer "B.Cu") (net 3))
 (segment (start 158.6697 130.3839) (end 160.3861 130.3839) (width 0.2) (layer "B.Cu") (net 3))
 (segment (start 152 134) (end 152.9019 134) (width 0.2) (layer "B.Cu") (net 3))
 (segment (start 152.9019 134.6764) (end 153.4362 135.2107) (width 0.2) (layer "B.Cu") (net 3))
 (segment (start 156.6883 133.1336) (end 156.6883 132.3653) (width 0.2) (layer "B.Cu") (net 3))
 (segment (start 156.6883 132.3653) (end 158.6697 130.3839) (width 0.2) (layer "B.Cu") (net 3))
 (segment (start 153.4362 135.2107) (end 154.6112 135.2107) (width 0.2) (layer "B.Cu") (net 3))
 (segment (start 152.9019 134) (end 152.9019 134.6764) (width 0.2) (layer "B.Cu") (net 3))
 (segment (start 152.9625 112.0875) (end 152.9625 111) (width 0.5) (layer "F.Cu") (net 8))
 (segment (start 147.6 117.45) (end 152.9625 112.0875) (width 0.5) (layer "F.Cu") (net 8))
 (segment (start 160.6925 118.73) (end 159 117.0375) (width 0.5) (layer "F.Cu") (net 17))
 (segment (start 166 118.73) (end 160.6925 118.73) (width 0.5) (layer "F.Cu") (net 17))
 (segment (start 136.7675 121.27) (end 141 117.0375) (width 0.5) (layer "F.Cu") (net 2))
 (segment (start 134 121.27) (end 136.7675 121.27) (width 0.5) (layer "F.Cu") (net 2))
 (segment (start 150.9375 120.8744) (end 150.9375 120.5375) (width 0.5) (layer "F.Cu") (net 11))
 (segment (start 150.9375 120.5375) (end 152.4 119.075) (width 0.5) (layer "F.Cu") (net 11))
 (segment (start 150.9375 123) (end 150.9375 120.8744) (width 0.5) (layer "F.Cu") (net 11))
 (via (at 150.9375 120.8744) (size 0.6) (drill 0.3) (layers "F.Cu" "B.Cu") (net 11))
 (segment (start 147.4208 109.1511) (end 147.4208 120.637) (width 0.5) (layer "B.Cu") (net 11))
 (segment (start 150.9375 120.8744) (end 147.6582 120.8744) (width 0.5) (layer "B.Cu") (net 11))
 (segment (start 144.9411 123.5915) (end 144.9411 134.7139) (width 0.5) (layer "B.Cu") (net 11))
 (segment (start 151.27 105.3019) (end 147.4208 109.1511) (width 0.5) (layer "B.Cu") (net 11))
 (segment (start 147.6582 120.8744) (end 144.9411 123.5915) (width 0.5) (layer "B.Cu") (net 11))
 (segment (start 151.27 104) (end 151.27 105.3019) (width 0.5) (layer "B.Cu") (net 11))
 (segment (start 146.2272 136) (end 148.73 136) (width 0.5) (layer "B.Cu") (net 11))
 (segment (start 147.4208 120.637) (end 147.6582 120.8744) (width 0.5) (layer "B.Cu") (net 11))
 (segment (start 144.9411 134.7139) (end 146.2272 136) (width 0.5) (layer "B.Cu") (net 11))
 (segment (start 153.3356 124.7769) (end 154.2 123.9125) (width 0.2) (layer "F.Cu") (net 15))
 (segment (start 153.2166 124.7769) (end 153.3356 124.7769) (width 0.2) (layer "F.Cu") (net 15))
 (via (at 153.2166 124.7769) (size 0.6) (drill 0.3) (layers "F.Cu" "B.Cu") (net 15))
 (segment (start 148 134) (end 148.9019 134) (width 0.2) (layer "B.Cu") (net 15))
 (segment (start 148.9019 129.0916) (end 153.2166 124.7769) (width 0.2) (layer "B.Cu") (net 15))
 (segment (start 148.9019 134) (end 148.9019 129.0916) (width 0.2) (layer "B.Cu") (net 15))
 (segment (start 149.9746 119.075) (end 147.6 119.075) (width 0.2) (layer "F.Cu") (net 9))
 (segment (start 151.5996 117.45) (end 149.9746 119.075) (width 0.2) (layer "F.Cu") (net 9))
 (segment (start 152.4 117.45) (end 151.5996 117.45) (width 0.2) (layer "F.Cu") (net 9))
 (segment (start 155.3233 102.8481) (end 150.7457 102.8481) (width 0.2) (layer "B.Cu") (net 10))
 (segment (start 149.8819 103.7119) (end 149.8819 104) (width 0.2) (layer "B.Cu") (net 10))
 (segment (start 166 120.1181) (end 165.208 120.1181) (width 0.2) (layer "B.Cu") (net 10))
 (segment (start 150.7457 102.8481) (end 149.8819 103.7119) (width 0.2) (layer "B.Cu") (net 10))
 (segment (start 165.208 120.1181) (end 164.8481 119.7582) (width 0.2) (layer "B.Cu") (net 10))
 (segment (start 164.8481 112.3729) (end 155.3233 102.8481) (width 0.2) (layer "B.Cu") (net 10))
 (segment (start 148.73 104) (end 149.8819 104) (width 0.2) (layer "B.Cu") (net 10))
 (segment (start 164.8481 119.7582) (end 164.8481 112.3729) (width 0.2) (layer "B.Cu") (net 10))
 (segment (start 166 121.27) (end 166 120.1181) (width 0.2) (layer "B.Cu") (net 10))
 (segment (start 151.27 136) (end 150.1181 136) (width 0.2) (layer "B.Cu") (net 14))
 (segment (start 134.7919 119.8819) (end 144.0004 129.0904) (width 0.2) (layer "B.Cu") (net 14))
 (segment (start 150.1181 136.2881) (end 150.1181 136) (width 0.2) (layer "B.Cu") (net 14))
 (segment (start 134 119.8819) (end 134.7919 119.8819) (width 0.2) (layer "B.Cu") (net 14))
 (segment (start 134 118.73) (end 134 119.8819) (width 0.2) (layer "B.Cu") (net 14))
 (segment (start 144.0004 129.0904) (end 144.0004 134.5585) (width 0.2) (layer "B.Cu") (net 14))
 (segment (start 144.0004 134.5585) (end 146.5938 137.1519) (width 0.2) (layer "B.Cu") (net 14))
 (segment (start 146.5938 137.1519) (end 149.2543 137.1519) (width 0.2) (layer "B.Cu") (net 14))
 (segment (start 149.2543 137.1519) (end 150.1181 136.2881) (width 0.2) (layer "B.Cu") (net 14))
 (segment (start 149.0625 122.5624) (end 150.1225 123.6224) (width 0.2) (layer "F.Cu") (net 16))
 (segment (start 152.6651 123.6224) (end 154.2 122.0875) (width 0.2) (layer "F.Cu") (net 16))
 (segment (start 149.0625 122.05) (end 149.0625 122.5624) (width 0.2) (layer "F.Cu") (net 16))
 (segment (start 150.1225 123.6224) (end 152.6651 123.6224) (width 0.2) (layer "F.Cu") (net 16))
 (segment (start 158.9467 113.3867) (end 160.9234 111.41) (width 0.2) (layer "F.Cu") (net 13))
 (segment (start 160.9234 111.41) (end 162.18 111.41) (width 0.2) (layer "F.Cu") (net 13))
 (segment (start 143.3867 109.7967) (end 143.3867 111.0533) (width 0.2) (layer "F.Cu") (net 7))
 (segment (start 141.41 107.82) (end 143.3867 109.7967) (width 0.2) (layer "F.Cu") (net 7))
 (segment (start 139.0746 128.59) (end 137.82 128.59) (width 0.2) (layer "F.Cu") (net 12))
 (segment (start 141.0533 126.6133) (end 139.1678 128.4988) (width 0.2) (layer "F.Cu") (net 12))
 (segment (start 139.1658 128.4988) (end 139.0746 128.59) (width 0.2) (layer "F.Cu") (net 12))
 (segment (start 139.1678 128.4988) (end 139.1658 128.4988) (width 0.2) (layer "F.Cu") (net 12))
 (segment (start 156.6133 130.2033) (end 156.6133 128.9467) (width 0.2) (layer "F.Cu") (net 5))
 (segment (start 158.59 132.18) (end 156.6133 130.2033) (width 0.2) (layer "F.Cu") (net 5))
 (segment (start 154 134) (end 150.475 130.475) (width 0.5) (layer "F.Cu") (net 1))
 (segment (start 150 130.3482) (end 142.6143 122.9625) (width 0.5) (layer "F.Cu") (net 1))
 (segment (start 159 122.9625) (end 156.1379 122.9625) (width 0.5) (layer "F.Cu") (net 1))
 (segment (start 150 130.475) (end 150 130.3482) (width 0.5) (layer "F.Cu") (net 1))
 (segment (start 142.6143 122.9625) (end 141 122.9625) (width 0.5) (layer "F.Cu") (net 1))
 (segment (start 148.0524 112.0149) (end 147.0375 111) (width 0.5) (layer "F.Cu") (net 1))
 (segment (start 150.475 130.475) (end 150 130.475) (width 0.5) (layer "F.Cu") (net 1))
 (segment (start 148.1727 112.0149) (end 148.0524 112.0149) (width 0.5) (layer "F.Cu") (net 1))
 (via (at 148.1727 112.0149) (size 0.6) (drill 0.3) (layers "F.Cu" "B.Cu") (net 1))
 (via (at 156.1379 122.9625) (size 0.6) (drill 0.3) (layers "F.Cu" "B.Cu") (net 1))
 (segment (start 156.1379 122.9625) (end 156.1379 119.9801) (width 0.5) (layer "B.Cu") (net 1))
 (segment (start 156.1379 131.8621) (end 156.1379 122.9625) (width 0.5) (layer "B.Cu") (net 1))
 (segment (start 156.1379 119.9801) (end 148.1727 112.0149) (width 0.5) (layer "B.Cu") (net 1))
 (segment (start 154 134) (end 156.1379 131.8621) (width 0.5) (layer "B.Cu") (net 1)))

